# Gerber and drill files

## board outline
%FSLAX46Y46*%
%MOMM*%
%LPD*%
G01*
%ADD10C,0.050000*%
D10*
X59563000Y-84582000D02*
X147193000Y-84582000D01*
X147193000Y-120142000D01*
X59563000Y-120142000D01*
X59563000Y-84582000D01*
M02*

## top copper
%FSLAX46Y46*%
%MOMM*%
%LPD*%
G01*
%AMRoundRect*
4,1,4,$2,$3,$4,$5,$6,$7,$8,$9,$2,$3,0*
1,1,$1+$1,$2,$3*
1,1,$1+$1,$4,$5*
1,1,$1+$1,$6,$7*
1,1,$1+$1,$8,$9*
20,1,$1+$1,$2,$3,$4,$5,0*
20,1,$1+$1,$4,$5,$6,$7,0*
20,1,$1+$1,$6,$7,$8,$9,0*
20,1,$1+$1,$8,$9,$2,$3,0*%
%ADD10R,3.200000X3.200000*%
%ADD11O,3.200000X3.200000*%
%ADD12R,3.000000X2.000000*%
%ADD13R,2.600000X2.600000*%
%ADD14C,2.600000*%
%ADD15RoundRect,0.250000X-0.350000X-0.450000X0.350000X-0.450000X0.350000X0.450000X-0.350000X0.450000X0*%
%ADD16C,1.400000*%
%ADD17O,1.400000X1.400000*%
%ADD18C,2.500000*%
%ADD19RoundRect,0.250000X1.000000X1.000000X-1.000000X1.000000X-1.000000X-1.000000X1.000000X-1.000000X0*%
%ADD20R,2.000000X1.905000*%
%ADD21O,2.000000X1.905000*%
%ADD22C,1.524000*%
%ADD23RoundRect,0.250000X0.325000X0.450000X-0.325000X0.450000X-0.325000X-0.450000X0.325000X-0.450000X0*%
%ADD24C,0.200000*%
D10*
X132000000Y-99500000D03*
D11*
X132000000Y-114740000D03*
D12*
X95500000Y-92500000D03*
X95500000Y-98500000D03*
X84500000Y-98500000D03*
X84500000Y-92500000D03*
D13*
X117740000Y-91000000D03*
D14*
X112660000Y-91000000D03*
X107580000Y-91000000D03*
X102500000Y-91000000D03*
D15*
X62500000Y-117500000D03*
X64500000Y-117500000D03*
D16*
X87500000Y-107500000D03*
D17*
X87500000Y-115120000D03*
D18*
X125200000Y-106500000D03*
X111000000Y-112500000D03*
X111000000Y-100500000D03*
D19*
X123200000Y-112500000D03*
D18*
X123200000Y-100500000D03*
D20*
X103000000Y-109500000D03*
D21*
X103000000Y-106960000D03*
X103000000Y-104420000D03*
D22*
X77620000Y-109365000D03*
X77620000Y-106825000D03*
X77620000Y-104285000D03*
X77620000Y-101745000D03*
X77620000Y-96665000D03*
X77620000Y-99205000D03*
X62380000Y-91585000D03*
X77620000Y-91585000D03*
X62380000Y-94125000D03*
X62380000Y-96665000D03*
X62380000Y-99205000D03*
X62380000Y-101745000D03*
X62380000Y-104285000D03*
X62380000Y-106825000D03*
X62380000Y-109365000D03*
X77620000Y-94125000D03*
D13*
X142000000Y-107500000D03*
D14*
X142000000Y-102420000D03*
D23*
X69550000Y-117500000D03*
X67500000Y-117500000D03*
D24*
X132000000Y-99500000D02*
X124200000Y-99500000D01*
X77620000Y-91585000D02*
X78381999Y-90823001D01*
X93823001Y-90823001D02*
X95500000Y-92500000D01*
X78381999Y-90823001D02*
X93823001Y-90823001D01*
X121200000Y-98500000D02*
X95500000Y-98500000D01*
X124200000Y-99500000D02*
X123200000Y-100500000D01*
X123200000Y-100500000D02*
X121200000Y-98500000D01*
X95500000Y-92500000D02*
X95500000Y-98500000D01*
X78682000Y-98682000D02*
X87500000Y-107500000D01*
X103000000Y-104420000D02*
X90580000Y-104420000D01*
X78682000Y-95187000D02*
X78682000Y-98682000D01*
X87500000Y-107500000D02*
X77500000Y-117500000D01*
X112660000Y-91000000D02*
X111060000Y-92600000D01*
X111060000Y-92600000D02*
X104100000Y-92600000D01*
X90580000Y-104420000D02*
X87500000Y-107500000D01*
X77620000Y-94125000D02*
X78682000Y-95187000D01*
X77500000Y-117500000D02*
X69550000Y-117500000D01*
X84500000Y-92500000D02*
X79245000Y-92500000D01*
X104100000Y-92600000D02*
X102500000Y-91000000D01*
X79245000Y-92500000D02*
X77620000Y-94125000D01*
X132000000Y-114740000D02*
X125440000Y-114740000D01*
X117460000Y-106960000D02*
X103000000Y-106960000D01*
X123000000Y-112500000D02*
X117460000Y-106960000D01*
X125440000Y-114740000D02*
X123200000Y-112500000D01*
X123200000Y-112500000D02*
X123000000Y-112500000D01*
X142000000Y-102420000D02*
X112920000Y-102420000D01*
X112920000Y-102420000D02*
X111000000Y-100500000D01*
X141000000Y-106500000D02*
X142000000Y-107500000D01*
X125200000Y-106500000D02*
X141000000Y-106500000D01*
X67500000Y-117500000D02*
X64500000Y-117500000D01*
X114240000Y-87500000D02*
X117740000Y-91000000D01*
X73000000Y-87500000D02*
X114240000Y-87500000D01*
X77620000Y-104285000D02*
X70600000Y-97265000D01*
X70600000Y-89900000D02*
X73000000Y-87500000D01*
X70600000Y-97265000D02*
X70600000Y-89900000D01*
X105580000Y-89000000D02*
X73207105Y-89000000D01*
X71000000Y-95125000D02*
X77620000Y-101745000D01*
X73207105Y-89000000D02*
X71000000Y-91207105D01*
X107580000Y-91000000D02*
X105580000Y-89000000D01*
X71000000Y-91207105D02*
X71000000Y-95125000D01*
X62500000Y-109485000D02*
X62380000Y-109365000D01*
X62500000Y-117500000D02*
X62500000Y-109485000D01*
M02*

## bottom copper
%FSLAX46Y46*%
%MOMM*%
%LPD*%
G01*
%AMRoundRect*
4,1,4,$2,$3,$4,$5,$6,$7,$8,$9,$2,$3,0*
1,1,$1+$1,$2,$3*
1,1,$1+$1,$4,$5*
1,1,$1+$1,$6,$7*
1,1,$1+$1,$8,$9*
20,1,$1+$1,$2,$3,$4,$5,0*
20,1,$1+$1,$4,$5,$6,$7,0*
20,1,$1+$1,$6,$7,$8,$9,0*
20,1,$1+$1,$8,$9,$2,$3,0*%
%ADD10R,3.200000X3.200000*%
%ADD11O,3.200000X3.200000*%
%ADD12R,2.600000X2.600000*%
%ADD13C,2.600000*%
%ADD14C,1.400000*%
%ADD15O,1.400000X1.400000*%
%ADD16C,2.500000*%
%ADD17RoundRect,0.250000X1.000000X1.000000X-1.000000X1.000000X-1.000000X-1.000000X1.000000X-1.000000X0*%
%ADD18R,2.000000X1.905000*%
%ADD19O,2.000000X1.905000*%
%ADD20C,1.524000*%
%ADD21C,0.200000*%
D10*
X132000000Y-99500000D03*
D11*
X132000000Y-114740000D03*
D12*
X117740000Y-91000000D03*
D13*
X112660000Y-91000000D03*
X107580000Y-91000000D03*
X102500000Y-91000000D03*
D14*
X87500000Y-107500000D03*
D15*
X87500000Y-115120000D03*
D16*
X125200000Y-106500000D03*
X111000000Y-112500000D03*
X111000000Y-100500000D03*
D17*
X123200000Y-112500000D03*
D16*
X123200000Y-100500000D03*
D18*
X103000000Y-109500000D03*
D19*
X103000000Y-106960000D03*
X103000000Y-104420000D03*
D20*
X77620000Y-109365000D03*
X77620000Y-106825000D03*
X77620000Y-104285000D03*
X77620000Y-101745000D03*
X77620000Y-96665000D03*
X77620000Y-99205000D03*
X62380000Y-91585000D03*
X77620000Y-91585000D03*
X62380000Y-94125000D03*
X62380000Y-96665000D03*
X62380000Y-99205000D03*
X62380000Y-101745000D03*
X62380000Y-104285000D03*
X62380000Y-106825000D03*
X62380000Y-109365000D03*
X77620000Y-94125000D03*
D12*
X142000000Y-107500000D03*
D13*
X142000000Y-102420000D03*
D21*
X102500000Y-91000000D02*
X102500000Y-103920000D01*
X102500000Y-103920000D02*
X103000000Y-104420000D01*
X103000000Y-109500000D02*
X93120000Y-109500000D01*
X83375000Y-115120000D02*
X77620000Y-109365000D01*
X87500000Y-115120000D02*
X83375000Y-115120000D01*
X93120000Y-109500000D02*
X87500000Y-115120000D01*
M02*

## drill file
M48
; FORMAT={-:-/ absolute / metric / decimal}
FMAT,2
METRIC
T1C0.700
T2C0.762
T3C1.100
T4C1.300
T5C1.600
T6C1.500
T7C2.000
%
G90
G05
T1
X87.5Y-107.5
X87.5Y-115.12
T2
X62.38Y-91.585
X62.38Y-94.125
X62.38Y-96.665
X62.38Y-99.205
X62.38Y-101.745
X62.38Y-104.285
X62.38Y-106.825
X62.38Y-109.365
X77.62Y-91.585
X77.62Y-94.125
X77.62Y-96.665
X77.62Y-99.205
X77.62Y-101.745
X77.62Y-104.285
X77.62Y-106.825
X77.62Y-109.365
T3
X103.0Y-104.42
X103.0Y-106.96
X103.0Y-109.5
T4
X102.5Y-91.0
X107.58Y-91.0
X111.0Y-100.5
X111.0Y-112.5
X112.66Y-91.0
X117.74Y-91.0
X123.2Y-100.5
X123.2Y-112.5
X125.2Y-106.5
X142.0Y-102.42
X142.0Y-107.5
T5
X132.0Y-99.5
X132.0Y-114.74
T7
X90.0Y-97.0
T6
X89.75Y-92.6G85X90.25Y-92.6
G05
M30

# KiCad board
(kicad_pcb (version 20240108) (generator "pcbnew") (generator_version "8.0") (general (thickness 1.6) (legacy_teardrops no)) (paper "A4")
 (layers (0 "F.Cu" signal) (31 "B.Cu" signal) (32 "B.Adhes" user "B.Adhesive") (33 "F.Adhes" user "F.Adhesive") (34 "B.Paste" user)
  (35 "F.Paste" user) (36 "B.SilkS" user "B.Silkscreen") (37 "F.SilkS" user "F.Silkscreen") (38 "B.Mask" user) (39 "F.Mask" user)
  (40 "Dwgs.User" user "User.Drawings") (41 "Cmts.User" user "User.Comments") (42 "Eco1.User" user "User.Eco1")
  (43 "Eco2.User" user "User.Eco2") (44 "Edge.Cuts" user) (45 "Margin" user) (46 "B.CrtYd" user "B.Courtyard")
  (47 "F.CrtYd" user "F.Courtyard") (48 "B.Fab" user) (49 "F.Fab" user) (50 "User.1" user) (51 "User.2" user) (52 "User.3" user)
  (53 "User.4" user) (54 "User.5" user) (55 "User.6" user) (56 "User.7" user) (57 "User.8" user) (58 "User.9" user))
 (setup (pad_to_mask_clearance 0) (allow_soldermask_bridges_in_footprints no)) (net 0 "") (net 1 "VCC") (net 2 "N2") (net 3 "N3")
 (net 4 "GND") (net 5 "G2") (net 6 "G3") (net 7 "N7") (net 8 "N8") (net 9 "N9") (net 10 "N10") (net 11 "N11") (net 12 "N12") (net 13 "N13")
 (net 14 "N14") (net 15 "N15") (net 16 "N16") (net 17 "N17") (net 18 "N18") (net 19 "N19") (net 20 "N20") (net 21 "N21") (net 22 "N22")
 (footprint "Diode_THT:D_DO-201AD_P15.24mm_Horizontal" (layer "F.Cu") (at 132 99.5 -90)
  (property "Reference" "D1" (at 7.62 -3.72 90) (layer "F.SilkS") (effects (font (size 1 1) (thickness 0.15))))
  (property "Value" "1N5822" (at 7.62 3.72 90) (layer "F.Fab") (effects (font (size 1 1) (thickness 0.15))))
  (pad "1" thru_hole rect (at 0 0 270) (size 3.2 3.2) (drill 1.6) (layers "*.Cu" "*.Mask") (remove_unused_layers no) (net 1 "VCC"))
  (pad "2" thru_hole oval (at 15.24 0 270) (size 3.2 3.2) (drill 1.6) (layers "*.Cu" "*.Mask") (remove_unused_layers no) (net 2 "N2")))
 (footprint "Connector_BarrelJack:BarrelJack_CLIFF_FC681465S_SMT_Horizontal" (layer "F.Cu") (at 90 95.5 -90)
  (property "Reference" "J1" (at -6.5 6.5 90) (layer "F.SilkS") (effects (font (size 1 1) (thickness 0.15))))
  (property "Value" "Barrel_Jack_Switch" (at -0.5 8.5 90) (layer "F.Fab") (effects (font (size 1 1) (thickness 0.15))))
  (pad "" np_thru_hole oval (at -2.9 0) (size 2 1.5) (drill oval 2 1.5) (layers "*.Cu" "*.Mask"))
  (pad "" np_thru_hole circle (at 1.5 0) (size 2 2) (drill 2) (layers "*.Cu" "*.Mask"))
  (pad "1" smd rect (at -3 -5.5) (size 3 2) (layers "F.Cu" "F.Paste" "F.Mask") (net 1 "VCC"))
  (pad "1" smd rect (at 3 -5.5) (size 3 2) (layers "F.Cu" "F.Paste" "F.Mask") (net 1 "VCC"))
  (pad "2" smd rect (at 3 5.5) (size 3 2) (layers "F.Cu" "F.Paste" "F.Mask") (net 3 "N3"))
  (pad "3" smd rect (at -3 5.5) (size 3 2) (layers "F.Cu" "F.Paste" "F.Mask") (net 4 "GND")))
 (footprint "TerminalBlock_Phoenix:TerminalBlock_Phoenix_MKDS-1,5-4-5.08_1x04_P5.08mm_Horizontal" (layer "F.Cu") (at 117.74 91 180)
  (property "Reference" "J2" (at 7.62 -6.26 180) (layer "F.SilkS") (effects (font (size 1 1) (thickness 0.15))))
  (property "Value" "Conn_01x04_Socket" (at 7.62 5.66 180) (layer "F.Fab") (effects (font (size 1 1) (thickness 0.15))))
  (pad "1" thru_hole rect (at 0 0 180) (size 2.6 2.6) (drill 1.3) (layers "*.Cu" "*.Mask") (remove_unused_layers no) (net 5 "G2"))
  (pad "2" thru_hole circle (at 5.08 0 180) (size 2.6 2.6) (drill 1.3) (layers "*.Cu" "*.Mask") (remove_unused_layers no) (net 4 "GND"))
  (pad "3" thru_hole circle (at 10.16 0 180) (size 2.6 2.6) (drill 1.3) (layers "*.Cu" "*.Mask") (remove_unused_layers no) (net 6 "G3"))
  (pad "4" thru_hole circle (at 15.24 0 180) (size 2.6 2.6) (drill 1.3) (layers "*.Cu" "*.Mask") (remove_unused_layers no) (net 4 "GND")))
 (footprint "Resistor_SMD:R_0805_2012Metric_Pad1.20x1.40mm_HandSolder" (layer "F.Cu") (at 63.5 117.5)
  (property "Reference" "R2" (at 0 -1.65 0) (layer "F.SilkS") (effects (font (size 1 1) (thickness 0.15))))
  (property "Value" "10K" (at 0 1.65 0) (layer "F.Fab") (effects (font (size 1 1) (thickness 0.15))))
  (pad "1" smd roundrect (at -1 0) (size 1.2 1.4) (layers "F.Cu" "F.Paste" "F.Mask") (roundrect_rratio 0.208333) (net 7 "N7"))
  (pad "2" smd roundrect (at 1 0) (size 1.2 1.4) (layers "F.Cu" "F.Paste" "F.Mask") (roundrect_rratio 0.208333) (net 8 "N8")))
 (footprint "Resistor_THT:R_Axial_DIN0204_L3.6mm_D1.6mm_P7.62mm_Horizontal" (layer "F.Cu") (at 87.5 107.5 -90)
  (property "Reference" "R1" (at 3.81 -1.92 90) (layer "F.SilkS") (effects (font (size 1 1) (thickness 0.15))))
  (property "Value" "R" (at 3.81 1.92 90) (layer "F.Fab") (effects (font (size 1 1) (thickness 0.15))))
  (pad "1" thru_hole circle (at 0 0 270) (size 1.4 1.4) (drill 0.7) (layers "*.Cu" "*.Mask") (remove_unused_layers no) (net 4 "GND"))
  (pad "2" thru_hole oval (at 7.62 0 270) (size 1.4 1.4) (drill 0.7) (layers "*.Cu" "*.Mask") (remove_unused_layers no) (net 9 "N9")))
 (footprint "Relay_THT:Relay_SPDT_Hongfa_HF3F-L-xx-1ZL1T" (layer "F.Cu") (at 123.2 112.5 180)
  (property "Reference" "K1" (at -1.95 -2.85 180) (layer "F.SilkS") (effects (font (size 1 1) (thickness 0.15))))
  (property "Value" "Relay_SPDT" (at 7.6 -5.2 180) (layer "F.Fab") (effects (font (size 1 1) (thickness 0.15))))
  (pad "11" thru_hole circle (at -2 6 180) (size 2.5 2.5) (drill 1.3) (layers "*.Cu" "*.Mask") (remove_unused_layers no) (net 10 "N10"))
  (pad "12" thru_hole circle (at 12.2 0 180) (size 2.5 2.5) (drill 1.3) (layers "*.Cu" "*.Mask") (remove_unused_layers no) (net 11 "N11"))
  (pad "14" thru_hole circle (at 12.2 12 180) (size 2.5 2.5) (drill 1.3) (layers "*.Cu" "*.Mask") (remove_unused_layers no) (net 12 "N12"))
  (pad "A1" thru_hole roundrect (at 0 0 180) (size 2.5 2.5) (drill 1.3) (layers "*.Cu" "*.Mask") (remove_unused_layers no)
   (roundrect_rratio 0.1) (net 2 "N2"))
  (pad "A2" thru_hole circle (at 0 12 180) (size 2.5 2.5) (drill 1.3) (layers "*.Cu" "*.Mask") (remove_unused_layers no) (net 1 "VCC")))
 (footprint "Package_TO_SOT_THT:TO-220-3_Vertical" (layer "F.Cu") (at 103 109.5 90)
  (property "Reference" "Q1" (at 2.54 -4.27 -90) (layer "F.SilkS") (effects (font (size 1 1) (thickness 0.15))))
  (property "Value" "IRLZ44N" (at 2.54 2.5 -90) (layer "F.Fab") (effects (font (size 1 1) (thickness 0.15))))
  (pad "1" thru_hole rect (at 0 0 90) (size 1.905 2) (drill 1.1) (layers "*.Cu" "*.Mask") (remove_unused_layers no) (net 9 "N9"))
  (pad "2" thru_hole oval (at 2.54 0 90) (size 1.905 2) (drill 1.1) (layers "*.Cu" "*.Mask") (remove_unused_layers no) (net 2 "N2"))
  (pad "3" thru_hole oval (at 5.08 0 90) (size 1.905 2) (drill 1.1) (layers "*.Cu" "*.Mask") (remove_unused_layers no) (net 4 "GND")))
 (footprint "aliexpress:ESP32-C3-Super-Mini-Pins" (layer "F.Cu") (at 70 99.205)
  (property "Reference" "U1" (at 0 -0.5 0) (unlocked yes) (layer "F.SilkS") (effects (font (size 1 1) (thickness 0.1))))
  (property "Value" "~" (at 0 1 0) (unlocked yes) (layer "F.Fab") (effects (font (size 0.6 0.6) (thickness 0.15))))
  (pad "0" thru_hole circle (at 7.62 10.16) (size 1.524 1.524) (drill 0.762) (layers "*.Cu" "*.Mask") (remove_unused_layers no) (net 9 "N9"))
  (pad "1" thru_hole circle (at 7.62 7.62) (size 1.524 1.524) (drill 0.762) (layers "*.Cu" "*.Mask") (remove_unused_layers no)
   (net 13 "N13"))
  (pad "2" thru_hole circle (at 7.62 5.08) (size 1.524 1.524) (drill 0.762) (layers "*.Cu" "*.Mask") (remove_unused_layers no) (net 5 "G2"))
  (pad "3" thru_hole circle (at 7.62 2.54) (size 1.524 1.524) (drill 0.762) (layers "*.Cu" "*.Mask") (remove_unused_layers no) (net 6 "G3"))
  (pad "3V3" thru_hole circle (at 7.62 -2.54) (size 1.524 1.524) (drill 0.762) (layers "*.Cu" "*.Mask") (remove_unused_layers no)
   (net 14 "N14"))
  (pad "4" thru_hole circle (at 7.62 0) (size 1.524 1.524) (drill 0.762) (layers "*.Cu" "*.Mask") (remove_unused_layers no) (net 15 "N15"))
  (pad "5" thru_hole circle (at -7.62 -7.62) (size 1.524 1.524) (drill 0.762) (layers "*.Cu" "*.Mask") (remove_unused_layers no)
   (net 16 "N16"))
  (pad "5V" thru_hole circle (at 7.62 -7.62) (size 1.524 1.524) (drill 0.762) (layers "*.Cu" "*.Mask") (remove_unused_layers no)
   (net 1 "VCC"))
  (pad "6" thru_hole circle (at -7.62 -5.08) (size 1.524 1.524) (drill 0.762) (layers "*.Cu" "*.Mask") (remove_unused_layers no)
   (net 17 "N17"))
  (pad "7" thru_hole circle (at -7.62 -2.54) (size 1.524 1.524) (drill 0.762) (layers "*.Cu" "*.Mask") (remove_unused_layers no)
   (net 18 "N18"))
  (pad "8" thru_hole circle (at -7.62 0) (size 1.524 1.524) (drill 0.762) (layers "*.Cu" "*.Mask") (remove_unused_layers no) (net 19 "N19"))
  (pad "9" thru_hole circle (at -7.62 2.54) (size 1.524 1.524) (drill 0.762) (layers "*.Cu" "*.Mask") (remove_unused_layers no)
   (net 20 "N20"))
  (pad "10" thru_hole circle (at -7.62 5.08) (size 1.524 1.524) (drill 0.762) (layers "*.Cu" "*.Mask") (remove_unused_layers no)
   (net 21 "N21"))
  (pad "20" thru_hole circle (at -7.62 7.62) (size 1.524 1.524) (drill 0.762) (layers "*.Cu" "*.Mask") (remove_unused_layers no)
   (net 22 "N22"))
  (pad "21" thru_hole circle (at -7.62 10.16) (size 1.524 1.524) (drill 0.762) (layers "*.Cu" "*.Mask") (remove_unused_layers no)
   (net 7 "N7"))
  (pad "G" thru_hole circle (at 7.62 -5.08) (size 1.524 1.524) (drill 0.762) (layers "*.Cu" "*.Mask") (remove_unused_layers no)
   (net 4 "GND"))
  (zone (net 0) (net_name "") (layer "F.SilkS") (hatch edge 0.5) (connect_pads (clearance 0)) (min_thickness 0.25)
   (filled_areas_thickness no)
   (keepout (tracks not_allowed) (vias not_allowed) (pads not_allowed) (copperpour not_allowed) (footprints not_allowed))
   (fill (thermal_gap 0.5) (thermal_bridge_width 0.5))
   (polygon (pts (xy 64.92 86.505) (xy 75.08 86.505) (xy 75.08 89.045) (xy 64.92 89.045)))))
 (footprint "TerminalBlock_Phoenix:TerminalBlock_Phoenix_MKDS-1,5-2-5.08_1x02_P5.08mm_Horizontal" (layer "F.Cu") (at 142 107.5 90)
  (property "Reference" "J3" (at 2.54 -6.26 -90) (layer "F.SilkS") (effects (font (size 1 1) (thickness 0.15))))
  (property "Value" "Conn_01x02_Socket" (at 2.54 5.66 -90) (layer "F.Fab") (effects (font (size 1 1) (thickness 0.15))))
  (pad "1" thru_hole rect (at 0 0 90) (size 2.6 2.6) (drill 1.3) (layers "*.Cu" "*.Mask") (remove_unused_layers no) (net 10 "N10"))
  (pad "2" thru_hole circle (at 5.08 0 90) (size 2.6 2.6) (drill 1.3) (layers "*.Cu" "*.Mask") (remove_unused_layers no) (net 12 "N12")))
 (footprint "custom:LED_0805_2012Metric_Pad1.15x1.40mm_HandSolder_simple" (layer "F.Cu") (at 68.525 117.5 180)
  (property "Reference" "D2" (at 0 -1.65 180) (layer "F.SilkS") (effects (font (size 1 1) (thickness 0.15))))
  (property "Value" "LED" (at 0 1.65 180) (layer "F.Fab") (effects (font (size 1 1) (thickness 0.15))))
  (pad "1" smd roundrect (at -1.025 0 180) (size 1.15 1.4) (layers "F.Cu" "F.Paste" "F.Mask") (roundrect_rratio 0.217391) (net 4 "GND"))
  (pad "2" smd roundrect (at 1.025 0 180) (size 1.15 1.4) (layers "F.Cu" "F.Paste" "F.Mask") (roundrect_rratio 0.217391) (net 8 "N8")))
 (gr_rect (start 59.563 84.582) (end 147.193 120.142) (stroke (width 0.05) (type default)) (fill none) (layer "Edge.Cuts"))
 (segment (start 132 99.5) (end 124.2 99.5) (width 0.2) (layer "F.Cu") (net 1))
 (segment (start 77.62 91.585) (end 78.381999 90.823001) (width 0.2) (layer "F.Cu") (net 1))
 (segment (start 93.823001 90.823001) (end 95.5 92.5) (width 0.2) (layer "F.Cu") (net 1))
 (segment (start 78.381999 90.823001) (end 93.823001 90.823001) (width 0.2) (layer "F.Cu") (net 1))
 (segment (start 121.2 98.5) (end 95.5 98.5) (width 0.2) (layer "F.Cu") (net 1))
 (segment (start 124.2 99.5) (end 123.2 100.5) (width 0.2) (layer "F.Cu") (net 1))
 (segment (start 123.2 100.5) (end 121.2 98.5) (width 0.2) (layer "F.Cu") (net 1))
 (segment (start 95.5 92.5) (end 95.5 98.5) (width 0.2) (layer "F.Cu") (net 1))
 (segment (start 78.682 98.682) (end 87.5 107.5) (width 0.2) (layer "F.Cu") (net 4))
 (segment (start 103 104.42) (end 90.58 104.42) (width 0.2) (layer "F.Cu") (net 4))
 (segment (start 78.682 95.187) (end 78.682 98.682) (width 0.2) (layer "F.Cu") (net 4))
 (segment (start 87.5 107.5) (end 77.5 117.5) (width 0.2) (layer "F.Cu") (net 4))
 (segment (start 112.66 91) (end 111.06 92.6) (width 0.2) (layer "F.Cu") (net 4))
 (segment (start 111.06 92.6) (end 104.1 92.6) (width 0.2) (layer "F.Cu") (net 4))
 (segment (start 90.58 104.42) (end 87.5 107.5) (width 0.2) (layer "F.Cu") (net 4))
 (segment (start 77.62 94.125) (end 78.682 95.187) (width 0.2) (layer "F.Cu") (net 4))
 (segment (start 77.5 117.5) (end 69.55 117.5) (width 0.2) (layer "F.Cu") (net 4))
 (segment (start 84.5 92.5) (end 79.245 92.5) (width 0.2) (layer "F.Cu") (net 4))
 (segment (start 104.1 92.6) (end 102.5 91) (width 0.2) (layer "F.Cu") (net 4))
 (segment (start 79.245 92.5) (end 77.62 94.125) (width 0.2) (layer "F.Cu") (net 4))
 (segment (start 102.5 91) (end 102.5 103.92) (width 0.2) (layer "B.Cu") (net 4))
 (segment (start 102.5 103.92) (end 103 104.42) (width 0.2) (layer "B.Cu") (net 4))
 (segment (start 132 114.74) (end 125.44 114.74) (width 0.2) (layer "F.Cu") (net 2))
 (segment (start 117.46 106.96) (end 103 106.96) (width 0.2) (layer "F.Cu") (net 2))
 (segment (start 123 112.5) (end 117.46 106.96) (width 0.2) (layer "F.Cu") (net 2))
 (segment (start 125.44 114.74) (end 123.2 112.5) (width 0.2) (layer "F.Cu") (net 2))
 (segment (start 123.2 112.5) (end 123 112.5) (width 0.2) (layer "F.Cu") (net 2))
 (segment (start 142 102.42) (end 112.92 102.42) (width 0.2) (layer "F.Cu") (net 12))
 (segment (start 112.92 102.42) (end 111 100.5) (width 0.2) (layer "F.Cu") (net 12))
 (segment (start 141 106.5) (end 142 107.5) (width 0.2) (layer "F.Cu") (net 10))
 (segment (start 125.2 106.5) (end 141 106.5) (width 0.2) (layer "F.Cu") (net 10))
 (segment (start 103 109.5) (end 93.12 109.5) (width 0.2) (layer "B.Cu") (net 9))
 (segment (start 83.375 115.12) (end 77.62 109.365) (width 0.2) (layer "B.Cu") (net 9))
 (segment (start 87.5 115.12) (end 83.375 115.12) (width 0.2) (layer "B.Cu") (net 9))
 (segment (start 93.12 109.5) (end 87.5 115.12) (width 0.2) (layer "B.Cu") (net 9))
 (segment (start 67.5 117.5) (end 64.5 117.5) (width 0.2) (layer "F.Cu") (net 8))
 (segment (start 114.24 87.5) (end 117.74 91) (width 0.2) (layer "F.Cu") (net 5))
 (segment (start 73 87.5) (end 114.24 87.5) (width 0.2) (layer "F.Cu") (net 5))
 (segment (start 77.62 104.285) (end 70.6 97.265) (width 0.2) (layer "F.Cu") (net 5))
 (segment (start 70.6 89.9) (end 73 87.5) (width 0.2) (layer "F.Cu") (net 5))
 (segment (start 70.6 97.265) (end 70.6 89.9) (width 0.2) (layer "F.Cu") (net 5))
 (segment (start 105.58 89) (end 73.207105 89) (width 0.2) (layer "F.Cu") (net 6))
 (segment (start 71 95.125) (end 77.62 101.745) (width 0.2) (layer "F.Cu") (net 6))
 (segment (start 73.207105 89) (end 71 91.207105) (width 0.2) (layer "F.Cu") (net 6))
 (segment (start 107.58 91) (end 105.58 89) (width 0.2) (layer "F.Cu") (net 6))
 (segment (start 71 91.207105) (end 71 95.125) (width 0.2) (layer "F.Cu") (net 6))
 (segment (start 62.5 109.485) (end 62.38 109.365) (width 0.2) (layer "F.Cu") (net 7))
 (segment (start 62.5 117.5) (end 62.5 109.485) (width 0.2) (layer "F.Cu") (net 7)))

